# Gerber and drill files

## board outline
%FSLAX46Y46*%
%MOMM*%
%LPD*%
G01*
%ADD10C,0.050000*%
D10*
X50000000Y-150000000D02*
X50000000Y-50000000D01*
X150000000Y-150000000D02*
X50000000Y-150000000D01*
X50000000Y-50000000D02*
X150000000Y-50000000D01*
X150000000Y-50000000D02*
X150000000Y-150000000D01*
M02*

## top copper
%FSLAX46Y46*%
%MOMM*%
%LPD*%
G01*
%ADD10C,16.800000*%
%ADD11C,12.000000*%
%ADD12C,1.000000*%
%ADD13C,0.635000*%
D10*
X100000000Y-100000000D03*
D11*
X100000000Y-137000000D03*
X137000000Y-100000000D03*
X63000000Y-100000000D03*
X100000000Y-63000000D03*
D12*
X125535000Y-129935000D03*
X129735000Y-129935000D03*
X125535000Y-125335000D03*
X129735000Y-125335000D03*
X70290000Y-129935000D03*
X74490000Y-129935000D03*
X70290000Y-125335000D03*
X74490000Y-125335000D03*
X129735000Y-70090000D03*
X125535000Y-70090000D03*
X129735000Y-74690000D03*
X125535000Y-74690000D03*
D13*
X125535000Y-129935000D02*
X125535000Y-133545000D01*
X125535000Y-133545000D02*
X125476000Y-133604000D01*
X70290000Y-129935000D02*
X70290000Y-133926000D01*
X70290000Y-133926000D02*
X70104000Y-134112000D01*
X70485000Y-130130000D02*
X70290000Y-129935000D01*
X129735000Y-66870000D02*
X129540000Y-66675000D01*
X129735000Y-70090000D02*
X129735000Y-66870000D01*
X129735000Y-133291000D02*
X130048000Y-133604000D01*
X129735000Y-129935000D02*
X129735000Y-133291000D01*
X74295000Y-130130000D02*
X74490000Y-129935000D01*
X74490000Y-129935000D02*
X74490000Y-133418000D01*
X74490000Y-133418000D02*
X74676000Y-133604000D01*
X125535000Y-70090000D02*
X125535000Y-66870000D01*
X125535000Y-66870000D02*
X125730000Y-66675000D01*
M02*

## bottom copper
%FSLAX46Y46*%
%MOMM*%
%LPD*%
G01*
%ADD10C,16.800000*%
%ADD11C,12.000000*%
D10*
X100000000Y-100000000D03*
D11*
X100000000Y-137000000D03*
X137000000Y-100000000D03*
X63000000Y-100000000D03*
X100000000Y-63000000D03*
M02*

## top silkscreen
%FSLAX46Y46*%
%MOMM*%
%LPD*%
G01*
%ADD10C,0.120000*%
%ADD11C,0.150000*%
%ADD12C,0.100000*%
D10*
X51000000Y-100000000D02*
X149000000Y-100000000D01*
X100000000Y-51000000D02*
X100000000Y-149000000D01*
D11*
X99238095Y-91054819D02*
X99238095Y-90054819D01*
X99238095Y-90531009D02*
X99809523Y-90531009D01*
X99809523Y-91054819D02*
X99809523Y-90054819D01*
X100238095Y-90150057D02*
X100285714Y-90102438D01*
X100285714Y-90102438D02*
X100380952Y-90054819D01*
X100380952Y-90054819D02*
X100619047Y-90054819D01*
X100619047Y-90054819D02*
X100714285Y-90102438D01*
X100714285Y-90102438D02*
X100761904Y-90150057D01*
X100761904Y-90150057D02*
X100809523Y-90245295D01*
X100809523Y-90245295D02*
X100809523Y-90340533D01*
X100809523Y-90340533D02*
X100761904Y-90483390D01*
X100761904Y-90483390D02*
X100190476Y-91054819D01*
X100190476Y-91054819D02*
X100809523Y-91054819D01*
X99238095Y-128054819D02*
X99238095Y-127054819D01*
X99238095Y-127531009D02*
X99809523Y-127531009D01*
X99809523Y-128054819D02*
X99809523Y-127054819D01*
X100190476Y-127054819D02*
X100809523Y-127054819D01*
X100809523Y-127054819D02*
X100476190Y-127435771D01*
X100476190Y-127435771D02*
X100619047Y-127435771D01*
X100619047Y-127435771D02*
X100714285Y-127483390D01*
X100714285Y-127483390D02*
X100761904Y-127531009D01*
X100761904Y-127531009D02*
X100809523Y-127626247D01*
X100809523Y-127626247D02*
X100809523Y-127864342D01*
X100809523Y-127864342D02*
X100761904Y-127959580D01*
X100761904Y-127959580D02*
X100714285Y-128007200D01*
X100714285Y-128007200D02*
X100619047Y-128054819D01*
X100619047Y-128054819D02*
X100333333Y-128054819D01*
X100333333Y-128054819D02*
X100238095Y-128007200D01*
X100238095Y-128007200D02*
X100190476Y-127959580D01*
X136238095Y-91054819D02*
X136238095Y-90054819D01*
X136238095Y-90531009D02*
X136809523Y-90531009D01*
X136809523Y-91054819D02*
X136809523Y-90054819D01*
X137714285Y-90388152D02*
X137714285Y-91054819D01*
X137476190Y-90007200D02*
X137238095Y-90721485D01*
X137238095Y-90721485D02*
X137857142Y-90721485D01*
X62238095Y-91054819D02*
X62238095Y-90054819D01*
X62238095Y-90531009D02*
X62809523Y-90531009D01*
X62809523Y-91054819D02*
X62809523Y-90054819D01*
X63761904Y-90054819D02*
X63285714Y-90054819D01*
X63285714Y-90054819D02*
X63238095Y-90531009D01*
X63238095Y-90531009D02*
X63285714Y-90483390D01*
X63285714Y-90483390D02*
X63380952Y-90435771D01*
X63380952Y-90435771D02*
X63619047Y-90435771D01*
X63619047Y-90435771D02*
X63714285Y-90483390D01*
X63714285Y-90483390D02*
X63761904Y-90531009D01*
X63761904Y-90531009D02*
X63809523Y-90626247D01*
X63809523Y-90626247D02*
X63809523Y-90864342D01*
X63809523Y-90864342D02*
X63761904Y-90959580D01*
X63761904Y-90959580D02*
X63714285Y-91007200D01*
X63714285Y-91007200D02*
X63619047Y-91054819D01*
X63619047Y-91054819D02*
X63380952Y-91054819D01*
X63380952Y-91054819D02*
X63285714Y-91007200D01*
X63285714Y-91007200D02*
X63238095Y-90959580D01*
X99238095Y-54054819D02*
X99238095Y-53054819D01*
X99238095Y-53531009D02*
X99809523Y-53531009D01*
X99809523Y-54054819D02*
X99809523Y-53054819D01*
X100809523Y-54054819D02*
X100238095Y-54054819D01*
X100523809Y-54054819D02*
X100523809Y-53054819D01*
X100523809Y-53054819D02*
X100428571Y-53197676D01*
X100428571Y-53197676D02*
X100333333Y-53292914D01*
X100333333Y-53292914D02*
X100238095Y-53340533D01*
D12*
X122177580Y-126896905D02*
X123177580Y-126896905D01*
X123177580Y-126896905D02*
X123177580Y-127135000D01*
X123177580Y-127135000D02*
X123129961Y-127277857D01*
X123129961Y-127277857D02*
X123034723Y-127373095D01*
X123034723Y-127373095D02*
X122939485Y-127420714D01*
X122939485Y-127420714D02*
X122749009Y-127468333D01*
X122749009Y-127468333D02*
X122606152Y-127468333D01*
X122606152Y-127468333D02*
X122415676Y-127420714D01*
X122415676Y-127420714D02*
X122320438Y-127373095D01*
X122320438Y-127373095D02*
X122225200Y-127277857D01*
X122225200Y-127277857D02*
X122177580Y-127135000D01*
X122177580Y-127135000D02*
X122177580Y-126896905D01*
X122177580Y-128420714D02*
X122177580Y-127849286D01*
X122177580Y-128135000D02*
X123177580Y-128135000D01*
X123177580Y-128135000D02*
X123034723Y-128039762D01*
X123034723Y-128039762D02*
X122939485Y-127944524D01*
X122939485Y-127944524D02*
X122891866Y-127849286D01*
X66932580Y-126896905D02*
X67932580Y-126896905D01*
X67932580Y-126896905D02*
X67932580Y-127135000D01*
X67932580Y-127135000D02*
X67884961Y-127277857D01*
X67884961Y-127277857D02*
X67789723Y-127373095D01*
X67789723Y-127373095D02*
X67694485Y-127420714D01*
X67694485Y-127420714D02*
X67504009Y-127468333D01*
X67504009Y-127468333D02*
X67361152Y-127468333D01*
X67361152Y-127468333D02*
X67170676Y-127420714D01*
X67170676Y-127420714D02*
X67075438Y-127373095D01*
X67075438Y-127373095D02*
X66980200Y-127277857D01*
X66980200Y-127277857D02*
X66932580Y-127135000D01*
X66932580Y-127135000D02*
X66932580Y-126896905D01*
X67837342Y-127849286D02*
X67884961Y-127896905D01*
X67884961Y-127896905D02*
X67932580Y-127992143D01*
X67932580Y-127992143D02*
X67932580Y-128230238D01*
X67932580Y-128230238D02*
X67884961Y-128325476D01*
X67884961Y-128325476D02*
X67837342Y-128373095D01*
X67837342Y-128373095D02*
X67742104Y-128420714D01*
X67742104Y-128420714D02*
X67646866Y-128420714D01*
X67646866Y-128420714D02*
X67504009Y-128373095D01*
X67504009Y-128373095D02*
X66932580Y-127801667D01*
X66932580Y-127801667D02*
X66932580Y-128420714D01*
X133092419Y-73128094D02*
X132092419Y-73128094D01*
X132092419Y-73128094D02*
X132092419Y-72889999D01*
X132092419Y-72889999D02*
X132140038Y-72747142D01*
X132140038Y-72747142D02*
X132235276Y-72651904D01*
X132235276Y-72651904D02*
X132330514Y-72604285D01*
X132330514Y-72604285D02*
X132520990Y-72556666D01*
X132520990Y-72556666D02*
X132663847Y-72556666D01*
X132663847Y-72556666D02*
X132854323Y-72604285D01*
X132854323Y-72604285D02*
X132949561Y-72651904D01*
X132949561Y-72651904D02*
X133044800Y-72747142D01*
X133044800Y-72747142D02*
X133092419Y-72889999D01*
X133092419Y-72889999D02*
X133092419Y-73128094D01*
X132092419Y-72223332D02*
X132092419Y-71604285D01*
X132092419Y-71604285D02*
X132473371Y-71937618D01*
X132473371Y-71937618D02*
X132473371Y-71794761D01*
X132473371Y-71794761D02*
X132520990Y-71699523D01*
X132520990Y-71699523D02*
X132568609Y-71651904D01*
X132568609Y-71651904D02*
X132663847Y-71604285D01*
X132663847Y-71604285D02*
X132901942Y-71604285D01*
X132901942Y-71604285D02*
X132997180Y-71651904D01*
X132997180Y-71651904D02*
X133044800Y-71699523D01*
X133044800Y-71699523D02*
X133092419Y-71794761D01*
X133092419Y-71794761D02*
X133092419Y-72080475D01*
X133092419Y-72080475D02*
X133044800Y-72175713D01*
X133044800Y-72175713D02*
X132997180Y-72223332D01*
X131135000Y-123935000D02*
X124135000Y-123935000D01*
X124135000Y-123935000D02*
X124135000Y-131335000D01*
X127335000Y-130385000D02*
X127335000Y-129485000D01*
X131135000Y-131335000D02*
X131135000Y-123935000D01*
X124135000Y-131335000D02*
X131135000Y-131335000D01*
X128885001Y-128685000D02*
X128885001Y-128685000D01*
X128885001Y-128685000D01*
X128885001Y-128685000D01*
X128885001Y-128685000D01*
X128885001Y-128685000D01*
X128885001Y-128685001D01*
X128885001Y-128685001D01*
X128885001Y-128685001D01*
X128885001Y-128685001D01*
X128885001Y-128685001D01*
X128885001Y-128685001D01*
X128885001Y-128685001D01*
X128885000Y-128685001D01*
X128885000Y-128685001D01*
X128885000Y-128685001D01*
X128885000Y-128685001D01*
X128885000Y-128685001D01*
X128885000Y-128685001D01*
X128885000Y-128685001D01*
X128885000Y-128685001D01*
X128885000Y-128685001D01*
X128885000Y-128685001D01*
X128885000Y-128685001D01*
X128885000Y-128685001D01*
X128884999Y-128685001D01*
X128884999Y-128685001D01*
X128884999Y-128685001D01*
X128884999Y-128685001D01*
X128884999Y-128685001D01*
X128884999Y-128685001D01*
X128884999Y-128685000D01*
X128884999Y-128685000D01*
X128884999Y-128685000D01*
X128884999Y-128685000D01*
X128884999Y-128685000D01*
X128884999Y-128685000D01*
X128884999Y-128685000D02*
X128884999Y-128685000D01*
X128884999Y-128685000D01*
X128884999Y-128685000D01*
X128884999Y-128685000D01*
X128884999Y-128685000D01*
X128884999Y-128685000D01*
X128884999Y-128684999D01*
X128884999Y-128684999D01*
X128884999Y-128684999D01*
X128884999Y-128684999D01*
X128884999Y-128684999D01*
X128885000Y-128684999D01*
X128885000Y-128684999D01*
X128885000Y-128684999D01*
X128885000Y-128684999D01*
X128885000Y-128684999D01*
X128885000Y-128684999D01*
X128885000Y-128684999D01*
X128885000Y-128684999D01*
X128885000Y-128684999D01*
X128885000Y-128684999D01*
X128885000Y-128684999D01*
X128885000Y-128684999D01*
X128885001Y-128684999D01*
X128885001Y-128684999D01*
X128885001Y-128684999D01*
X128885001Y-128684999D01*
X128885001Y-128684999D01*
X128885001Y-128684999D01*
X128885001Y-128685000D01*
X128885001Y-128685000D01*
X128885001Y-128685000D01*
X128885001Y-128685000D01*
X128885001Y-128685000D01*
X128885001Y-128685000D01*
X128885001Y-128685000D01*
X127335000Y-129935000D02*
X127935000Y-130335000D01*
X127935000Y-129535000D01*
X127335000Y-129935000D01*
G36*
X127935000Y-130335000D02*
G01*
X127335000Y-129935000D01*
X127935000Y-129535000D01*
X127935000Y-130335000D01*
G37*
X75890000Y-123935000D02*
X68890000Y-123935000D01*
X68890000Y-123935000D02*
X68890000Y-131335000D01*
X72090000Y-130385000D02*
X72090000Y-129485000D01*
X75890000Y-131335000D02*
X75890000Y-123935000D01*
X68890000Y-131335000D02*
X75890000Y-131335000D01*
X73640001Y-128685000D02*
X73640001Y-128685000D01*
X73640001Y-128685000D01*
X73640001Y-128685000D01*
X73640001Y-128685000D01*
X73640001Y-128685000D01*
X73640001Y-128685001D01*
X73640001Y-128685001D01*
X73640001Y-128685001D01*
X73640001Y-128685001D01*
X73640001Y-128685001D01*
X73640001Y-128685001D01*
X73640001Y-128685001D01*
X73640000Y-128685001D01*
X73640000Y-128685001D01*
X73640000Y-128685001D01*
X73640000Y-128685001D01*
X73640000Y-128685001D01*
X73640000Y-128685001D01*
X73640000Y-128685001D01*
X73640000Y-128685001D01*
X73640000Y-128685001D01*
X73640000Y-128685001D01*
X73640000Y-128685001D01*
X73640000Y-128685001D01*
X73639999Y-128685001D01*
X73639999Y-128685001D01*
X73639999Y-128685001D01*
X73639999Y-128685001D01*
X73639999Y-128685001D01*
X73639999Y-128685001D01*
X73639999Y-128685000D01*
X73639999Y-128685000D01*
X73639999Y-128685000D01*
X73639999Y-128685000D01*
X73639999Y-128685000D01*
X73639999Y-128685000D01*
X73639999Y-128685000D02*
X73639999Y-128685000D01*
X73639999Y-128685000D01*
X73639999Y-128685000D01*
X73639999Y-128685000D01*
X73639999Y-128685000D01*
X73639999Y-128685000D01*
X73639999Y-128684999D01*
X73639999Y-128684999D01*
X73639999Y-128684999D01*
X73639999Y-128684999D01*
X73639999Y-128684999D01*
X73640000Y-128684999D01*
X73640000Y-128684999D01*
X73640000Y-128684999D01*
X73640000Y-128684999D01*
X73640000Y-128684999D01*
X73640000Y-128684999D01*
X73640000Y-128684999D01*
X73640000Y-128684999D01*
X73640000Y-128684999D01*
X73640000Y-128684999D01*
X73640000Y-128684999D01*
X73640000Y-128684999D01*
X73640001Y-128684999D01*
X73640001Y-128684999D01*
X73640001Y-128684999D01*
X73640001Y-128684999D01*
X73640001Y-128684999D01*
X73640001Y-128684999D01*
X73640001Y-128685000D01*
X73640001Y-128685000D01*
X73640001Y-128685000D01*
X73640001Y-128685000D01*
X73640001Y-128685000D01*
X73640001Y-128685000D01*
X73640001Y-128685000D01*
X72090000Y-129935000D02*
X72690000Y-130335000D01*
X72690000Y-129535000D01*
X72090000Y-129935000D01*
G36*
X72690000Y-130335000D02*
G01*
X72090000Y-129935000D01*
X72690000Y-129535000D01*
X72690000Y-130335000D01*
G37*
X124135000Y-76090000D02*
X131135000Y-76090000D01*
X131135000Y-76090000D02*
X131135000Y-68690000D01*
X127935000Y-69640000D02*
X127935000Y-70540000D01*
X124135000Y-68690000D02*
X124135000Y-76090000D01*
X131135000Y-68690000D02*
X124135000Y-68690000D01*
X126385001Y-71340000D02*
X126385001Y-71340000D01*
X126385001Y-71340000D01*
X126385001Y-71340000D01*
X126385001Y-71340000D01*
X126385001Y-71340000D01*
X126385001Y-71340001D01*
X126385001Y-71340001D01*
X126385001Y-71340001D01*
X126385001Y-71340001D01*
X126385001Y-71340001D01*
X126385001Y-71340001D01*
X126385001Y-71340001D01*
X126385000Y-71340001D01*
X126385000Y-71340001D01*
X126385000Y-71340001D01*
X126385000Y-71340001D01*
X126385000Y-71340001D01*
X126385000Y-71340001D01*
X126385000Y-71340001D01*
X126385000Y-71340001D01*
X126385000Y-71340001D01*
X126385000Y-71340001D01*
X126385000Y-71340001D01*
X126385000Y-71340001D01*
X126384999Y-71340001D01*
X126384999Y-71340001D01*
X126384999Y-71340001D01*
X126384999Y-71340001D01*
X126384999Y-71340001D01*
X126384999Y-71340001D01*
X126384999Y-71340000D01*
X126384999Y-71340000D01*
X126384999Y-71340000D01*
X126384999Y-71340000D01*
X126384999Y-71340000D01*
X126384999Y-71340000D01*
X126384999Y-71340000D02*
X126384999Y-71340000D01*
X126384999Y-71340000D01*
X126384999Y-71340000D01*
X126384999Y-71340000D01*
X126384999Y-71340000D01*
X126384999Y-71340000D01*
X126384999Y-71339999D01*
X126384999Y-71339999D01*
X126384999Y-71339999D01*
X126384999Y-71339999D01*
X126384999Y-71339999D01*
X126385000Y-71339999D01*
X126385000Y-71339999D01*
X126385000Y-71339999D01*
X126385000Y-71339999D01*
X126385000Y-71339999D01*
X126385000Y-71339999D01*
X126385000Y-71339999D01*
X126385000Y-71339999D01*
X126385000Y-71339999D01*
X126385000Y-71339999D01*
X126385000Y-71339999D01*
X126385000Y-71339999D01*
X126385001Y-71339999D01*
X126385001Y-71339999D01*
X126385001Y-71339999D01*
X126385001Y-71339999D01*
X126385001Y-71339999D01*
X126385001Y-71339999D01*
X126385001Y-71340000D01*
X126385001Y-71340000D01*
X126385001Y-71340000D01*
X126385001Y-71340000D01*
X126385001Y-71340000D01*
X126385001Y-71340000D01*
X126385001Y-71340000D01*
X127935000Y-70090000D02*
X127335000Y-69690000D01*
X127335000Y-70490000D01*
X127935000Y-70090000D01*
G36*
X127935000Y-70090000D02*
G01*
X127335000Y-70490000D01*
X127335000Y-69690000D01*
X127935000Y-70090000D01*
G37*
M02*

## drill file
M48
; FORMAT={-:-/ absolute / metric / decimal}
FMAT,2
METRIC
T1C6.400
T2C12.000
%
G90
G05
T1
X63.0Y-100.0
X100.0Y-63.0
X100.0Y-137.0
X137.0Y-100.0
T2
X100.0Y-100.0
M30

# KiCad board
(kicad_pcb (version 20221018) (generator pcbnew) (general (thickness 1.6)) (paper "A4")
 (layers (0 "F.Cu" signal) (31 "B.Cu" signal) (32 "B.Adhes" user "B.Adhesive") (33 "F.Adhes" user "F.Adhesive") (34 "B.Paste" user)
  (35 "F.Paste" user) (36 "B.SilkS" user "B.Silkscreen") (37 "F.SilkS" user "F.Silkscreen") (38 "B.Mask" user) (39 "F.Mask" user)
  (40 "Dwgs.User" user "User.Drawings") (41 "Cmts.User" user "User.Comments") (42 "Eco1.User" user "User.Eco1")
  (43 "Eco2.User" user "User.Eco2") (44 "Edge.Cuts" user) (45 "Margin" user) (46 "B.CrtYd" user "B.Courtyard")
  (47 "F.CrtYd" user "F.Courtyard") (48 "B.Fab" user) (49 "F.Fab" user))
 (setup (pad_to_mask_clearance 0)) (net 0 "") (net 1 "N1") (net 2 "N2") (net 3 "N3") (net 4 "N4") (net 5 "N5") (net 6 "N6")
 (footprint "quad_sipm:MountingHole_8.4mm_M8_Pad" (layer "F.Cu") (at 100 100)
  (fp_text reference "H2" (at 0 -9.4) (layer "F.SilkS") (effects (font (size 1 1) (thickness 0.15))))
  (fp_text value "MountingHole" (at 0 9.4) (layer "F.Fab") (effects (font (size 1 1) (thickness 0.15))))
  (pad "1" thru_hole circle (at 0 0) (size 16.8 16.8) (drill 12) (layers "*.Cu" "*.Mask")))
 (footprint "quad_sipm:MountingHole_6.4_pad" (layer "F.Cu") (at 100 137)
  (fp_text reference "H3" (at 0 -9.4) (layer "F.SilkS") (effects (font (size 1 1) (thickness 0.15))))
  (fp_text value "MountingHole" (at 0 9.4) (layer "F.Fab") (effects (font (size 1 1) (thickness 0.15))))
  (pad "1" thru_hole circle (at 0 0) (size 12 12) (drill 6.4) (layers "*.Cu" "*.Mask")))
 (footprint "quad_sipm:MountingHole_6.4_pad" (layer "F.Cu") (at 137 100)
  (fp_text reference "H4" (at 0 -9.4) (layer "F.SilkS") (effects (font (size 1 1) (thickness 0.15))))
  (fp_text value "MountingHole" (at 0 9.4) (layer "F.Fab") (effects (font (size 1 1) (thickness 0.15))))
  (pad "1" thru_hole circle (at 0 0) (size 12 12) (drill 6.4) (layers "*.Cu" "*.Mask")))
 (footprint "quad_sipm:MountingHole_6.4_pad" (layer "F.Cu") (at 63 100)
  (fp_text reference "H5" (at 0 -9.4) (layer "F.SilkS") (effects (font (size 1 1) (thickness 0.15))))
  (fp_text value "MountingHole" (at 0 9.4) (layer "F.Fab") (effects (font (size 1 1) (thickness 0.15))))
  (pad "1" thru_hole circle (at 0 0) (size 12 12) (drill 6.4) (layers "*.Cu" "*.Mask")))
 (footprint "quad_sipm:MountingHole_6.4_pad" (layer "F.Cu") (at 100 63)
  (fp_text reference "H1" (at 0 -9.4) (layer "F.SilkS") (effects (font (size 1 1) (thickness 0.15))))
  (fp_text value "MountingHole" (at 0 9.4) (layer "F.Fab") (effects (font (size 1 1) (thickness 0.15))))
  (pad "1" thru_hole circle (at 0 0) (size 12 12) (drill 6.4) (layers "*.Cu" "*.Mask")))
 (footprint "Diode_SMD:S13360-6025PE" (layer "F.Cu") (at 127.635 127.635 -90)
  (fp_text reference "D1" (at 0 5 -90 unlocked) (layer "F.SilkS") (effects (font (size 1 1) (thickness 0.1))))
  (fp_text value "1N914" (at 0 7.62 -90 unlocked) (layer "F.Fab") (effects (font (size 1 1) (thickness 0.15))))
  (fp_line (start -3.7 -3.5) (end -3.7 3.5) (stroke (width 0.1) (type default)) (layer "F.SilkS"))
  (fp_line (start -3.7 3.5) (end 3.7 3.5) (stroke (width 0.1) (type default)) (layer "F.SilkS"))
  (fp_line (start 2.75 0.3) (end 1.85 0.3) (stroke (width 0.1) (type default)) (layer "F.SilkS"))
  (fp_line (start 3.7 -3.5) (end -3.7 -3.5) (stroke (width 0.1) (type default)) (layer "F.SilkS"))
  (fp_line (start 3.7 3.5) (end 3.7 -3.5) (stroke (width 0.1) (type default)) (layer "F.SilkS"))
  (fp_circle (center 1.05 -1.25) (end 1.05 -1.25) (stroke (width 0.1) (type default)) (fill none) (layer "F.SilkS"))
  (fp_poly (pts (xy 2.3 0.3) (xy 2.7 -0.3) (xy 1.9 -0.3)) (stroke (width 0.1) (type solid)) (fill solid) (layer "F.SilkS"))
  (pad "1" smd circle (at 2.3 2.1 270) (size 1 1) (layers "F.Cu" "F.Paste" "F.Mask") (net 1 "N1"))
  (pad "2" smd circle (at 2.3 -2.1 270) (size 1 1) (layers "F.Cu" "F.Paste" "F.Mask") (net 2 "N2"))
  (pad "3" smd circle (at -2.3 2.1 270) (size 1 1) (layers "F.Cu" "F.Paste" "F.Mask"))
  (pad "4" smd circle (at -2.3 -2.1 270) (size 1 1) (layers "F.Cu" "F.Paste" "F.Mask")))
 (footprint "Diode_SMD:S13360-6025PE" (layer "F.Cu") (at 72.39 127.635 -90)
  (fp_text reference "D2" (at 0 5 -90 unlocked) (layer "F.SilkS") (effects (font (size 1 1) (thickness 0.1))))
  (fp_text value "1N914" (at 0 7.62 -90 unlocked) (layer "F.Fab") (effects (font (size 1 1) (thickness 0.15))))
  (fp_line (start -3.7 -3.5) (end -3.7 3.5) (stroke (width 0.1) (type default)) (layer "F.SilkS"))
  (fp_line (start -3.7 3.5) (end 3.7 3.5) (stroke (width 0.1) (type default)) (layer "F.SilkS"))
  (fp_line (start 2.75 0.3) (end 1.85 0.3) (stroke (width 0.1) (type default)) (layer "F.SilkS"))
  (fp_line (start 3.7 -3.5) (end -3.7 -3.5) (stroke (width 0.1) (type default)) (layer "F.SilkS"))
  (fp_line (start 3.7 3.5) (end 3.7 -3.5) (stroke (width 0.1) (type default)) (layer "F.SilkS"))
  (fp_circle (center 1.05 -1.25) (end 1.05 -1.25) (stroke (width 0.1) (type default)) (fill none) (layer "F.SilkS"))
  (fp_poly (pts (xy 2.3 0.3) (xy 2.7 -0.3) (xy 1.9 -0.3)) (stroke (width 0.1) (type solid)) (fill solid) (layer "F.SilkS"))
  (pad "1" smd circle (at 2.3 2.1 270) (size 1 1) (layers "F.Cu" "F.Paste" "F.Mask") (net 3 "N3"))
  (pad "2" smd circle (at 2.3 -2.1 270) (size 1 1) (layers "F.Cu" "F.Paste" "F.Mask") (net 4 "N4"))
  (pad "3" smd circle (at -2.3 2.1 270) (size 1 1) (layers "F.Cu" "F.Paste" "F.Mask"))
  (pad "4" smd circle (at -2.3 -2.1 270) (size 1 1) (layers "F.Cu" "F.Paste" "F.Mask")))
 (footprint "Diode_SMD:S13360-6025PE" (layer "F.Cu") (at 127.635 72.39 90)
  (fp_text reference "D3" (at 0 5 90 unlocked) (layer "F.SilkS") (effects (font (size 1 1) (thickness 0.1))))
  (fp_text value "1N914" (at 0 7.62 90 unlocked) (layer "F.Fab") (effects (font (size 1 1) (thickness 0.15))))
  (fp_line (start -3.7 -3.5) (end -3.7 3.5) (stroke (width 0.1) (type default)) (layer "F.SilkS"))
  (fp_line (start -3.7 3.5) (end 3.7 3.5) (stroke (width 0.1) (type default)) (layer "F.SilkS"))
  (fp_line (start 2.75 0.3) (end 1.85 0.3) (stroke (width 0.1) (type default)) (layer "F.SilkS"))
  (fp_line (start 3.7 -3.5) (end -3.7 -3.5) (stroke (width 0.1) (type default)) (layer "F.SilkS"))
  (fp_line (start 3.7 3.5) (end 3.7 -3.5) (stroke (width 0.1) (type default)) (layer "F.SilkS"))
  (fp_circle (center 1.05 -1.25) (end 1.05 -1.25) (stroke (width 0.1) (type default)) (fill none) (layer "F.SilkS"))
  (fp_poly (pts (xy 2.3 0.3) (xy 2.7 -0.3) (xy 1.9 -0.3)) (stroke (width 0.1) (type solid)) (fill solid) (layer "F.SilkS"))
  (pad "1" smd circle (at 2.3 2.1 90) (size 1 1) (layers "F.Cu" "F.Paste" "F.Mask") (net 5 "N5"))
  (pad "2" smd circle (at 2.3 -2.1 90) (size 1 1) (layers "F.Cu" "F.Paste" "F.Mask") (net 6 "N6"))
  (pad "3" smd circle (at -2.3 2.1 90) (size 1 1) (layers "F.Cu" "F.Paste" "F.Mask"))
  (pad "4" smd circle (at -2.3 -2.1 90) (size 1 1) (layers "F.Cu" "F.Paste" "F.Mask")))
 (gr_line (start 51 100) (end 149 100) (stroke (width 0.12) (type solid)) (layer "F.SilkS"))
 (gr_line (start 100 51) (end 100 149) (stroke (width 0.12) (type solid)) (layer "F.SilkS"))
 (gr_line (start 50 150) (end 50 50) (stroke (width 0.05) (type solid)) (layer "Edge.Cuts"))
 (gr_line (start 150 150) (end 50 150) (stroke (width 0.05) (type solid)) (layer "Edge.Cuts"))
 (gr_line (start 50 50) (end 150 50) (stroke (width 0.05) (type solid)) (layer "Edge.Cuts"))
 (gr_line (start 150 50) (end 150 150) (stroke (width 0.05) (type solid)) (layer "Edge.Cuts"))
 (segment (start 125.535 129.935) (end 125.535 133.545) (width 0.635) (layer "F.Cu") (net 1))
 (segment (start 125.535 133.545) (end 125.476 133.604) (width 0.635) (layer "F.Cu") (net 1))
 (segment (start 70.29 129.935) (end 70.29 133.926) (width 0.635) (layer "F.Cu") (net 3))
 (segment (start 70.29 133.926) (end 70.104 134.112) (width 0.635) (layer "F.Cu") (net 3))
 (segment (start 70.485 130.13) (end 70.29 129.935) (width 0.635) (layer "F.Cu") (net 3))
 (segment (start 129.735 66.87) (end 129.54 66.675) (width 0.635) (layer "F.Cu") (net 5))
 (segment (start 129.735 70.09) (end 129.735 66.87) (width 0.635) (layer "F.Cu") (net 5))
 (segment (start 129.735 133.291) (end 130.048 133.604) (width 0.635) (layer "F.Cu") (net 2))
 (segment (start 129.735 129.935) (end 129.735 133.291) (width 0.635) (layer "F.Cu") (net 2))
 (segment (start 74.295 130.13) (end 74.49 129.935) (width 0.635) (layer "F.Cu") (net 4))
 (segment (start 74.49 129.935) (end 74.49 133.418) (width 0.635) (layer "F.Cu") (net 4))
 (segment (start 74.49 133.418) (end 74.676 133.604) (width 0.635) (layer "F.Cu") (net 4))
 (segment (start 125.535 70.09) (end 125.535 66.87) (width 0.635) (layer "F.Cu") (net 6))
 (segment (start 125.535 66.87) (end 125.73 66.675) (width 0.635) (layer "F.Cu") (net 6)))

